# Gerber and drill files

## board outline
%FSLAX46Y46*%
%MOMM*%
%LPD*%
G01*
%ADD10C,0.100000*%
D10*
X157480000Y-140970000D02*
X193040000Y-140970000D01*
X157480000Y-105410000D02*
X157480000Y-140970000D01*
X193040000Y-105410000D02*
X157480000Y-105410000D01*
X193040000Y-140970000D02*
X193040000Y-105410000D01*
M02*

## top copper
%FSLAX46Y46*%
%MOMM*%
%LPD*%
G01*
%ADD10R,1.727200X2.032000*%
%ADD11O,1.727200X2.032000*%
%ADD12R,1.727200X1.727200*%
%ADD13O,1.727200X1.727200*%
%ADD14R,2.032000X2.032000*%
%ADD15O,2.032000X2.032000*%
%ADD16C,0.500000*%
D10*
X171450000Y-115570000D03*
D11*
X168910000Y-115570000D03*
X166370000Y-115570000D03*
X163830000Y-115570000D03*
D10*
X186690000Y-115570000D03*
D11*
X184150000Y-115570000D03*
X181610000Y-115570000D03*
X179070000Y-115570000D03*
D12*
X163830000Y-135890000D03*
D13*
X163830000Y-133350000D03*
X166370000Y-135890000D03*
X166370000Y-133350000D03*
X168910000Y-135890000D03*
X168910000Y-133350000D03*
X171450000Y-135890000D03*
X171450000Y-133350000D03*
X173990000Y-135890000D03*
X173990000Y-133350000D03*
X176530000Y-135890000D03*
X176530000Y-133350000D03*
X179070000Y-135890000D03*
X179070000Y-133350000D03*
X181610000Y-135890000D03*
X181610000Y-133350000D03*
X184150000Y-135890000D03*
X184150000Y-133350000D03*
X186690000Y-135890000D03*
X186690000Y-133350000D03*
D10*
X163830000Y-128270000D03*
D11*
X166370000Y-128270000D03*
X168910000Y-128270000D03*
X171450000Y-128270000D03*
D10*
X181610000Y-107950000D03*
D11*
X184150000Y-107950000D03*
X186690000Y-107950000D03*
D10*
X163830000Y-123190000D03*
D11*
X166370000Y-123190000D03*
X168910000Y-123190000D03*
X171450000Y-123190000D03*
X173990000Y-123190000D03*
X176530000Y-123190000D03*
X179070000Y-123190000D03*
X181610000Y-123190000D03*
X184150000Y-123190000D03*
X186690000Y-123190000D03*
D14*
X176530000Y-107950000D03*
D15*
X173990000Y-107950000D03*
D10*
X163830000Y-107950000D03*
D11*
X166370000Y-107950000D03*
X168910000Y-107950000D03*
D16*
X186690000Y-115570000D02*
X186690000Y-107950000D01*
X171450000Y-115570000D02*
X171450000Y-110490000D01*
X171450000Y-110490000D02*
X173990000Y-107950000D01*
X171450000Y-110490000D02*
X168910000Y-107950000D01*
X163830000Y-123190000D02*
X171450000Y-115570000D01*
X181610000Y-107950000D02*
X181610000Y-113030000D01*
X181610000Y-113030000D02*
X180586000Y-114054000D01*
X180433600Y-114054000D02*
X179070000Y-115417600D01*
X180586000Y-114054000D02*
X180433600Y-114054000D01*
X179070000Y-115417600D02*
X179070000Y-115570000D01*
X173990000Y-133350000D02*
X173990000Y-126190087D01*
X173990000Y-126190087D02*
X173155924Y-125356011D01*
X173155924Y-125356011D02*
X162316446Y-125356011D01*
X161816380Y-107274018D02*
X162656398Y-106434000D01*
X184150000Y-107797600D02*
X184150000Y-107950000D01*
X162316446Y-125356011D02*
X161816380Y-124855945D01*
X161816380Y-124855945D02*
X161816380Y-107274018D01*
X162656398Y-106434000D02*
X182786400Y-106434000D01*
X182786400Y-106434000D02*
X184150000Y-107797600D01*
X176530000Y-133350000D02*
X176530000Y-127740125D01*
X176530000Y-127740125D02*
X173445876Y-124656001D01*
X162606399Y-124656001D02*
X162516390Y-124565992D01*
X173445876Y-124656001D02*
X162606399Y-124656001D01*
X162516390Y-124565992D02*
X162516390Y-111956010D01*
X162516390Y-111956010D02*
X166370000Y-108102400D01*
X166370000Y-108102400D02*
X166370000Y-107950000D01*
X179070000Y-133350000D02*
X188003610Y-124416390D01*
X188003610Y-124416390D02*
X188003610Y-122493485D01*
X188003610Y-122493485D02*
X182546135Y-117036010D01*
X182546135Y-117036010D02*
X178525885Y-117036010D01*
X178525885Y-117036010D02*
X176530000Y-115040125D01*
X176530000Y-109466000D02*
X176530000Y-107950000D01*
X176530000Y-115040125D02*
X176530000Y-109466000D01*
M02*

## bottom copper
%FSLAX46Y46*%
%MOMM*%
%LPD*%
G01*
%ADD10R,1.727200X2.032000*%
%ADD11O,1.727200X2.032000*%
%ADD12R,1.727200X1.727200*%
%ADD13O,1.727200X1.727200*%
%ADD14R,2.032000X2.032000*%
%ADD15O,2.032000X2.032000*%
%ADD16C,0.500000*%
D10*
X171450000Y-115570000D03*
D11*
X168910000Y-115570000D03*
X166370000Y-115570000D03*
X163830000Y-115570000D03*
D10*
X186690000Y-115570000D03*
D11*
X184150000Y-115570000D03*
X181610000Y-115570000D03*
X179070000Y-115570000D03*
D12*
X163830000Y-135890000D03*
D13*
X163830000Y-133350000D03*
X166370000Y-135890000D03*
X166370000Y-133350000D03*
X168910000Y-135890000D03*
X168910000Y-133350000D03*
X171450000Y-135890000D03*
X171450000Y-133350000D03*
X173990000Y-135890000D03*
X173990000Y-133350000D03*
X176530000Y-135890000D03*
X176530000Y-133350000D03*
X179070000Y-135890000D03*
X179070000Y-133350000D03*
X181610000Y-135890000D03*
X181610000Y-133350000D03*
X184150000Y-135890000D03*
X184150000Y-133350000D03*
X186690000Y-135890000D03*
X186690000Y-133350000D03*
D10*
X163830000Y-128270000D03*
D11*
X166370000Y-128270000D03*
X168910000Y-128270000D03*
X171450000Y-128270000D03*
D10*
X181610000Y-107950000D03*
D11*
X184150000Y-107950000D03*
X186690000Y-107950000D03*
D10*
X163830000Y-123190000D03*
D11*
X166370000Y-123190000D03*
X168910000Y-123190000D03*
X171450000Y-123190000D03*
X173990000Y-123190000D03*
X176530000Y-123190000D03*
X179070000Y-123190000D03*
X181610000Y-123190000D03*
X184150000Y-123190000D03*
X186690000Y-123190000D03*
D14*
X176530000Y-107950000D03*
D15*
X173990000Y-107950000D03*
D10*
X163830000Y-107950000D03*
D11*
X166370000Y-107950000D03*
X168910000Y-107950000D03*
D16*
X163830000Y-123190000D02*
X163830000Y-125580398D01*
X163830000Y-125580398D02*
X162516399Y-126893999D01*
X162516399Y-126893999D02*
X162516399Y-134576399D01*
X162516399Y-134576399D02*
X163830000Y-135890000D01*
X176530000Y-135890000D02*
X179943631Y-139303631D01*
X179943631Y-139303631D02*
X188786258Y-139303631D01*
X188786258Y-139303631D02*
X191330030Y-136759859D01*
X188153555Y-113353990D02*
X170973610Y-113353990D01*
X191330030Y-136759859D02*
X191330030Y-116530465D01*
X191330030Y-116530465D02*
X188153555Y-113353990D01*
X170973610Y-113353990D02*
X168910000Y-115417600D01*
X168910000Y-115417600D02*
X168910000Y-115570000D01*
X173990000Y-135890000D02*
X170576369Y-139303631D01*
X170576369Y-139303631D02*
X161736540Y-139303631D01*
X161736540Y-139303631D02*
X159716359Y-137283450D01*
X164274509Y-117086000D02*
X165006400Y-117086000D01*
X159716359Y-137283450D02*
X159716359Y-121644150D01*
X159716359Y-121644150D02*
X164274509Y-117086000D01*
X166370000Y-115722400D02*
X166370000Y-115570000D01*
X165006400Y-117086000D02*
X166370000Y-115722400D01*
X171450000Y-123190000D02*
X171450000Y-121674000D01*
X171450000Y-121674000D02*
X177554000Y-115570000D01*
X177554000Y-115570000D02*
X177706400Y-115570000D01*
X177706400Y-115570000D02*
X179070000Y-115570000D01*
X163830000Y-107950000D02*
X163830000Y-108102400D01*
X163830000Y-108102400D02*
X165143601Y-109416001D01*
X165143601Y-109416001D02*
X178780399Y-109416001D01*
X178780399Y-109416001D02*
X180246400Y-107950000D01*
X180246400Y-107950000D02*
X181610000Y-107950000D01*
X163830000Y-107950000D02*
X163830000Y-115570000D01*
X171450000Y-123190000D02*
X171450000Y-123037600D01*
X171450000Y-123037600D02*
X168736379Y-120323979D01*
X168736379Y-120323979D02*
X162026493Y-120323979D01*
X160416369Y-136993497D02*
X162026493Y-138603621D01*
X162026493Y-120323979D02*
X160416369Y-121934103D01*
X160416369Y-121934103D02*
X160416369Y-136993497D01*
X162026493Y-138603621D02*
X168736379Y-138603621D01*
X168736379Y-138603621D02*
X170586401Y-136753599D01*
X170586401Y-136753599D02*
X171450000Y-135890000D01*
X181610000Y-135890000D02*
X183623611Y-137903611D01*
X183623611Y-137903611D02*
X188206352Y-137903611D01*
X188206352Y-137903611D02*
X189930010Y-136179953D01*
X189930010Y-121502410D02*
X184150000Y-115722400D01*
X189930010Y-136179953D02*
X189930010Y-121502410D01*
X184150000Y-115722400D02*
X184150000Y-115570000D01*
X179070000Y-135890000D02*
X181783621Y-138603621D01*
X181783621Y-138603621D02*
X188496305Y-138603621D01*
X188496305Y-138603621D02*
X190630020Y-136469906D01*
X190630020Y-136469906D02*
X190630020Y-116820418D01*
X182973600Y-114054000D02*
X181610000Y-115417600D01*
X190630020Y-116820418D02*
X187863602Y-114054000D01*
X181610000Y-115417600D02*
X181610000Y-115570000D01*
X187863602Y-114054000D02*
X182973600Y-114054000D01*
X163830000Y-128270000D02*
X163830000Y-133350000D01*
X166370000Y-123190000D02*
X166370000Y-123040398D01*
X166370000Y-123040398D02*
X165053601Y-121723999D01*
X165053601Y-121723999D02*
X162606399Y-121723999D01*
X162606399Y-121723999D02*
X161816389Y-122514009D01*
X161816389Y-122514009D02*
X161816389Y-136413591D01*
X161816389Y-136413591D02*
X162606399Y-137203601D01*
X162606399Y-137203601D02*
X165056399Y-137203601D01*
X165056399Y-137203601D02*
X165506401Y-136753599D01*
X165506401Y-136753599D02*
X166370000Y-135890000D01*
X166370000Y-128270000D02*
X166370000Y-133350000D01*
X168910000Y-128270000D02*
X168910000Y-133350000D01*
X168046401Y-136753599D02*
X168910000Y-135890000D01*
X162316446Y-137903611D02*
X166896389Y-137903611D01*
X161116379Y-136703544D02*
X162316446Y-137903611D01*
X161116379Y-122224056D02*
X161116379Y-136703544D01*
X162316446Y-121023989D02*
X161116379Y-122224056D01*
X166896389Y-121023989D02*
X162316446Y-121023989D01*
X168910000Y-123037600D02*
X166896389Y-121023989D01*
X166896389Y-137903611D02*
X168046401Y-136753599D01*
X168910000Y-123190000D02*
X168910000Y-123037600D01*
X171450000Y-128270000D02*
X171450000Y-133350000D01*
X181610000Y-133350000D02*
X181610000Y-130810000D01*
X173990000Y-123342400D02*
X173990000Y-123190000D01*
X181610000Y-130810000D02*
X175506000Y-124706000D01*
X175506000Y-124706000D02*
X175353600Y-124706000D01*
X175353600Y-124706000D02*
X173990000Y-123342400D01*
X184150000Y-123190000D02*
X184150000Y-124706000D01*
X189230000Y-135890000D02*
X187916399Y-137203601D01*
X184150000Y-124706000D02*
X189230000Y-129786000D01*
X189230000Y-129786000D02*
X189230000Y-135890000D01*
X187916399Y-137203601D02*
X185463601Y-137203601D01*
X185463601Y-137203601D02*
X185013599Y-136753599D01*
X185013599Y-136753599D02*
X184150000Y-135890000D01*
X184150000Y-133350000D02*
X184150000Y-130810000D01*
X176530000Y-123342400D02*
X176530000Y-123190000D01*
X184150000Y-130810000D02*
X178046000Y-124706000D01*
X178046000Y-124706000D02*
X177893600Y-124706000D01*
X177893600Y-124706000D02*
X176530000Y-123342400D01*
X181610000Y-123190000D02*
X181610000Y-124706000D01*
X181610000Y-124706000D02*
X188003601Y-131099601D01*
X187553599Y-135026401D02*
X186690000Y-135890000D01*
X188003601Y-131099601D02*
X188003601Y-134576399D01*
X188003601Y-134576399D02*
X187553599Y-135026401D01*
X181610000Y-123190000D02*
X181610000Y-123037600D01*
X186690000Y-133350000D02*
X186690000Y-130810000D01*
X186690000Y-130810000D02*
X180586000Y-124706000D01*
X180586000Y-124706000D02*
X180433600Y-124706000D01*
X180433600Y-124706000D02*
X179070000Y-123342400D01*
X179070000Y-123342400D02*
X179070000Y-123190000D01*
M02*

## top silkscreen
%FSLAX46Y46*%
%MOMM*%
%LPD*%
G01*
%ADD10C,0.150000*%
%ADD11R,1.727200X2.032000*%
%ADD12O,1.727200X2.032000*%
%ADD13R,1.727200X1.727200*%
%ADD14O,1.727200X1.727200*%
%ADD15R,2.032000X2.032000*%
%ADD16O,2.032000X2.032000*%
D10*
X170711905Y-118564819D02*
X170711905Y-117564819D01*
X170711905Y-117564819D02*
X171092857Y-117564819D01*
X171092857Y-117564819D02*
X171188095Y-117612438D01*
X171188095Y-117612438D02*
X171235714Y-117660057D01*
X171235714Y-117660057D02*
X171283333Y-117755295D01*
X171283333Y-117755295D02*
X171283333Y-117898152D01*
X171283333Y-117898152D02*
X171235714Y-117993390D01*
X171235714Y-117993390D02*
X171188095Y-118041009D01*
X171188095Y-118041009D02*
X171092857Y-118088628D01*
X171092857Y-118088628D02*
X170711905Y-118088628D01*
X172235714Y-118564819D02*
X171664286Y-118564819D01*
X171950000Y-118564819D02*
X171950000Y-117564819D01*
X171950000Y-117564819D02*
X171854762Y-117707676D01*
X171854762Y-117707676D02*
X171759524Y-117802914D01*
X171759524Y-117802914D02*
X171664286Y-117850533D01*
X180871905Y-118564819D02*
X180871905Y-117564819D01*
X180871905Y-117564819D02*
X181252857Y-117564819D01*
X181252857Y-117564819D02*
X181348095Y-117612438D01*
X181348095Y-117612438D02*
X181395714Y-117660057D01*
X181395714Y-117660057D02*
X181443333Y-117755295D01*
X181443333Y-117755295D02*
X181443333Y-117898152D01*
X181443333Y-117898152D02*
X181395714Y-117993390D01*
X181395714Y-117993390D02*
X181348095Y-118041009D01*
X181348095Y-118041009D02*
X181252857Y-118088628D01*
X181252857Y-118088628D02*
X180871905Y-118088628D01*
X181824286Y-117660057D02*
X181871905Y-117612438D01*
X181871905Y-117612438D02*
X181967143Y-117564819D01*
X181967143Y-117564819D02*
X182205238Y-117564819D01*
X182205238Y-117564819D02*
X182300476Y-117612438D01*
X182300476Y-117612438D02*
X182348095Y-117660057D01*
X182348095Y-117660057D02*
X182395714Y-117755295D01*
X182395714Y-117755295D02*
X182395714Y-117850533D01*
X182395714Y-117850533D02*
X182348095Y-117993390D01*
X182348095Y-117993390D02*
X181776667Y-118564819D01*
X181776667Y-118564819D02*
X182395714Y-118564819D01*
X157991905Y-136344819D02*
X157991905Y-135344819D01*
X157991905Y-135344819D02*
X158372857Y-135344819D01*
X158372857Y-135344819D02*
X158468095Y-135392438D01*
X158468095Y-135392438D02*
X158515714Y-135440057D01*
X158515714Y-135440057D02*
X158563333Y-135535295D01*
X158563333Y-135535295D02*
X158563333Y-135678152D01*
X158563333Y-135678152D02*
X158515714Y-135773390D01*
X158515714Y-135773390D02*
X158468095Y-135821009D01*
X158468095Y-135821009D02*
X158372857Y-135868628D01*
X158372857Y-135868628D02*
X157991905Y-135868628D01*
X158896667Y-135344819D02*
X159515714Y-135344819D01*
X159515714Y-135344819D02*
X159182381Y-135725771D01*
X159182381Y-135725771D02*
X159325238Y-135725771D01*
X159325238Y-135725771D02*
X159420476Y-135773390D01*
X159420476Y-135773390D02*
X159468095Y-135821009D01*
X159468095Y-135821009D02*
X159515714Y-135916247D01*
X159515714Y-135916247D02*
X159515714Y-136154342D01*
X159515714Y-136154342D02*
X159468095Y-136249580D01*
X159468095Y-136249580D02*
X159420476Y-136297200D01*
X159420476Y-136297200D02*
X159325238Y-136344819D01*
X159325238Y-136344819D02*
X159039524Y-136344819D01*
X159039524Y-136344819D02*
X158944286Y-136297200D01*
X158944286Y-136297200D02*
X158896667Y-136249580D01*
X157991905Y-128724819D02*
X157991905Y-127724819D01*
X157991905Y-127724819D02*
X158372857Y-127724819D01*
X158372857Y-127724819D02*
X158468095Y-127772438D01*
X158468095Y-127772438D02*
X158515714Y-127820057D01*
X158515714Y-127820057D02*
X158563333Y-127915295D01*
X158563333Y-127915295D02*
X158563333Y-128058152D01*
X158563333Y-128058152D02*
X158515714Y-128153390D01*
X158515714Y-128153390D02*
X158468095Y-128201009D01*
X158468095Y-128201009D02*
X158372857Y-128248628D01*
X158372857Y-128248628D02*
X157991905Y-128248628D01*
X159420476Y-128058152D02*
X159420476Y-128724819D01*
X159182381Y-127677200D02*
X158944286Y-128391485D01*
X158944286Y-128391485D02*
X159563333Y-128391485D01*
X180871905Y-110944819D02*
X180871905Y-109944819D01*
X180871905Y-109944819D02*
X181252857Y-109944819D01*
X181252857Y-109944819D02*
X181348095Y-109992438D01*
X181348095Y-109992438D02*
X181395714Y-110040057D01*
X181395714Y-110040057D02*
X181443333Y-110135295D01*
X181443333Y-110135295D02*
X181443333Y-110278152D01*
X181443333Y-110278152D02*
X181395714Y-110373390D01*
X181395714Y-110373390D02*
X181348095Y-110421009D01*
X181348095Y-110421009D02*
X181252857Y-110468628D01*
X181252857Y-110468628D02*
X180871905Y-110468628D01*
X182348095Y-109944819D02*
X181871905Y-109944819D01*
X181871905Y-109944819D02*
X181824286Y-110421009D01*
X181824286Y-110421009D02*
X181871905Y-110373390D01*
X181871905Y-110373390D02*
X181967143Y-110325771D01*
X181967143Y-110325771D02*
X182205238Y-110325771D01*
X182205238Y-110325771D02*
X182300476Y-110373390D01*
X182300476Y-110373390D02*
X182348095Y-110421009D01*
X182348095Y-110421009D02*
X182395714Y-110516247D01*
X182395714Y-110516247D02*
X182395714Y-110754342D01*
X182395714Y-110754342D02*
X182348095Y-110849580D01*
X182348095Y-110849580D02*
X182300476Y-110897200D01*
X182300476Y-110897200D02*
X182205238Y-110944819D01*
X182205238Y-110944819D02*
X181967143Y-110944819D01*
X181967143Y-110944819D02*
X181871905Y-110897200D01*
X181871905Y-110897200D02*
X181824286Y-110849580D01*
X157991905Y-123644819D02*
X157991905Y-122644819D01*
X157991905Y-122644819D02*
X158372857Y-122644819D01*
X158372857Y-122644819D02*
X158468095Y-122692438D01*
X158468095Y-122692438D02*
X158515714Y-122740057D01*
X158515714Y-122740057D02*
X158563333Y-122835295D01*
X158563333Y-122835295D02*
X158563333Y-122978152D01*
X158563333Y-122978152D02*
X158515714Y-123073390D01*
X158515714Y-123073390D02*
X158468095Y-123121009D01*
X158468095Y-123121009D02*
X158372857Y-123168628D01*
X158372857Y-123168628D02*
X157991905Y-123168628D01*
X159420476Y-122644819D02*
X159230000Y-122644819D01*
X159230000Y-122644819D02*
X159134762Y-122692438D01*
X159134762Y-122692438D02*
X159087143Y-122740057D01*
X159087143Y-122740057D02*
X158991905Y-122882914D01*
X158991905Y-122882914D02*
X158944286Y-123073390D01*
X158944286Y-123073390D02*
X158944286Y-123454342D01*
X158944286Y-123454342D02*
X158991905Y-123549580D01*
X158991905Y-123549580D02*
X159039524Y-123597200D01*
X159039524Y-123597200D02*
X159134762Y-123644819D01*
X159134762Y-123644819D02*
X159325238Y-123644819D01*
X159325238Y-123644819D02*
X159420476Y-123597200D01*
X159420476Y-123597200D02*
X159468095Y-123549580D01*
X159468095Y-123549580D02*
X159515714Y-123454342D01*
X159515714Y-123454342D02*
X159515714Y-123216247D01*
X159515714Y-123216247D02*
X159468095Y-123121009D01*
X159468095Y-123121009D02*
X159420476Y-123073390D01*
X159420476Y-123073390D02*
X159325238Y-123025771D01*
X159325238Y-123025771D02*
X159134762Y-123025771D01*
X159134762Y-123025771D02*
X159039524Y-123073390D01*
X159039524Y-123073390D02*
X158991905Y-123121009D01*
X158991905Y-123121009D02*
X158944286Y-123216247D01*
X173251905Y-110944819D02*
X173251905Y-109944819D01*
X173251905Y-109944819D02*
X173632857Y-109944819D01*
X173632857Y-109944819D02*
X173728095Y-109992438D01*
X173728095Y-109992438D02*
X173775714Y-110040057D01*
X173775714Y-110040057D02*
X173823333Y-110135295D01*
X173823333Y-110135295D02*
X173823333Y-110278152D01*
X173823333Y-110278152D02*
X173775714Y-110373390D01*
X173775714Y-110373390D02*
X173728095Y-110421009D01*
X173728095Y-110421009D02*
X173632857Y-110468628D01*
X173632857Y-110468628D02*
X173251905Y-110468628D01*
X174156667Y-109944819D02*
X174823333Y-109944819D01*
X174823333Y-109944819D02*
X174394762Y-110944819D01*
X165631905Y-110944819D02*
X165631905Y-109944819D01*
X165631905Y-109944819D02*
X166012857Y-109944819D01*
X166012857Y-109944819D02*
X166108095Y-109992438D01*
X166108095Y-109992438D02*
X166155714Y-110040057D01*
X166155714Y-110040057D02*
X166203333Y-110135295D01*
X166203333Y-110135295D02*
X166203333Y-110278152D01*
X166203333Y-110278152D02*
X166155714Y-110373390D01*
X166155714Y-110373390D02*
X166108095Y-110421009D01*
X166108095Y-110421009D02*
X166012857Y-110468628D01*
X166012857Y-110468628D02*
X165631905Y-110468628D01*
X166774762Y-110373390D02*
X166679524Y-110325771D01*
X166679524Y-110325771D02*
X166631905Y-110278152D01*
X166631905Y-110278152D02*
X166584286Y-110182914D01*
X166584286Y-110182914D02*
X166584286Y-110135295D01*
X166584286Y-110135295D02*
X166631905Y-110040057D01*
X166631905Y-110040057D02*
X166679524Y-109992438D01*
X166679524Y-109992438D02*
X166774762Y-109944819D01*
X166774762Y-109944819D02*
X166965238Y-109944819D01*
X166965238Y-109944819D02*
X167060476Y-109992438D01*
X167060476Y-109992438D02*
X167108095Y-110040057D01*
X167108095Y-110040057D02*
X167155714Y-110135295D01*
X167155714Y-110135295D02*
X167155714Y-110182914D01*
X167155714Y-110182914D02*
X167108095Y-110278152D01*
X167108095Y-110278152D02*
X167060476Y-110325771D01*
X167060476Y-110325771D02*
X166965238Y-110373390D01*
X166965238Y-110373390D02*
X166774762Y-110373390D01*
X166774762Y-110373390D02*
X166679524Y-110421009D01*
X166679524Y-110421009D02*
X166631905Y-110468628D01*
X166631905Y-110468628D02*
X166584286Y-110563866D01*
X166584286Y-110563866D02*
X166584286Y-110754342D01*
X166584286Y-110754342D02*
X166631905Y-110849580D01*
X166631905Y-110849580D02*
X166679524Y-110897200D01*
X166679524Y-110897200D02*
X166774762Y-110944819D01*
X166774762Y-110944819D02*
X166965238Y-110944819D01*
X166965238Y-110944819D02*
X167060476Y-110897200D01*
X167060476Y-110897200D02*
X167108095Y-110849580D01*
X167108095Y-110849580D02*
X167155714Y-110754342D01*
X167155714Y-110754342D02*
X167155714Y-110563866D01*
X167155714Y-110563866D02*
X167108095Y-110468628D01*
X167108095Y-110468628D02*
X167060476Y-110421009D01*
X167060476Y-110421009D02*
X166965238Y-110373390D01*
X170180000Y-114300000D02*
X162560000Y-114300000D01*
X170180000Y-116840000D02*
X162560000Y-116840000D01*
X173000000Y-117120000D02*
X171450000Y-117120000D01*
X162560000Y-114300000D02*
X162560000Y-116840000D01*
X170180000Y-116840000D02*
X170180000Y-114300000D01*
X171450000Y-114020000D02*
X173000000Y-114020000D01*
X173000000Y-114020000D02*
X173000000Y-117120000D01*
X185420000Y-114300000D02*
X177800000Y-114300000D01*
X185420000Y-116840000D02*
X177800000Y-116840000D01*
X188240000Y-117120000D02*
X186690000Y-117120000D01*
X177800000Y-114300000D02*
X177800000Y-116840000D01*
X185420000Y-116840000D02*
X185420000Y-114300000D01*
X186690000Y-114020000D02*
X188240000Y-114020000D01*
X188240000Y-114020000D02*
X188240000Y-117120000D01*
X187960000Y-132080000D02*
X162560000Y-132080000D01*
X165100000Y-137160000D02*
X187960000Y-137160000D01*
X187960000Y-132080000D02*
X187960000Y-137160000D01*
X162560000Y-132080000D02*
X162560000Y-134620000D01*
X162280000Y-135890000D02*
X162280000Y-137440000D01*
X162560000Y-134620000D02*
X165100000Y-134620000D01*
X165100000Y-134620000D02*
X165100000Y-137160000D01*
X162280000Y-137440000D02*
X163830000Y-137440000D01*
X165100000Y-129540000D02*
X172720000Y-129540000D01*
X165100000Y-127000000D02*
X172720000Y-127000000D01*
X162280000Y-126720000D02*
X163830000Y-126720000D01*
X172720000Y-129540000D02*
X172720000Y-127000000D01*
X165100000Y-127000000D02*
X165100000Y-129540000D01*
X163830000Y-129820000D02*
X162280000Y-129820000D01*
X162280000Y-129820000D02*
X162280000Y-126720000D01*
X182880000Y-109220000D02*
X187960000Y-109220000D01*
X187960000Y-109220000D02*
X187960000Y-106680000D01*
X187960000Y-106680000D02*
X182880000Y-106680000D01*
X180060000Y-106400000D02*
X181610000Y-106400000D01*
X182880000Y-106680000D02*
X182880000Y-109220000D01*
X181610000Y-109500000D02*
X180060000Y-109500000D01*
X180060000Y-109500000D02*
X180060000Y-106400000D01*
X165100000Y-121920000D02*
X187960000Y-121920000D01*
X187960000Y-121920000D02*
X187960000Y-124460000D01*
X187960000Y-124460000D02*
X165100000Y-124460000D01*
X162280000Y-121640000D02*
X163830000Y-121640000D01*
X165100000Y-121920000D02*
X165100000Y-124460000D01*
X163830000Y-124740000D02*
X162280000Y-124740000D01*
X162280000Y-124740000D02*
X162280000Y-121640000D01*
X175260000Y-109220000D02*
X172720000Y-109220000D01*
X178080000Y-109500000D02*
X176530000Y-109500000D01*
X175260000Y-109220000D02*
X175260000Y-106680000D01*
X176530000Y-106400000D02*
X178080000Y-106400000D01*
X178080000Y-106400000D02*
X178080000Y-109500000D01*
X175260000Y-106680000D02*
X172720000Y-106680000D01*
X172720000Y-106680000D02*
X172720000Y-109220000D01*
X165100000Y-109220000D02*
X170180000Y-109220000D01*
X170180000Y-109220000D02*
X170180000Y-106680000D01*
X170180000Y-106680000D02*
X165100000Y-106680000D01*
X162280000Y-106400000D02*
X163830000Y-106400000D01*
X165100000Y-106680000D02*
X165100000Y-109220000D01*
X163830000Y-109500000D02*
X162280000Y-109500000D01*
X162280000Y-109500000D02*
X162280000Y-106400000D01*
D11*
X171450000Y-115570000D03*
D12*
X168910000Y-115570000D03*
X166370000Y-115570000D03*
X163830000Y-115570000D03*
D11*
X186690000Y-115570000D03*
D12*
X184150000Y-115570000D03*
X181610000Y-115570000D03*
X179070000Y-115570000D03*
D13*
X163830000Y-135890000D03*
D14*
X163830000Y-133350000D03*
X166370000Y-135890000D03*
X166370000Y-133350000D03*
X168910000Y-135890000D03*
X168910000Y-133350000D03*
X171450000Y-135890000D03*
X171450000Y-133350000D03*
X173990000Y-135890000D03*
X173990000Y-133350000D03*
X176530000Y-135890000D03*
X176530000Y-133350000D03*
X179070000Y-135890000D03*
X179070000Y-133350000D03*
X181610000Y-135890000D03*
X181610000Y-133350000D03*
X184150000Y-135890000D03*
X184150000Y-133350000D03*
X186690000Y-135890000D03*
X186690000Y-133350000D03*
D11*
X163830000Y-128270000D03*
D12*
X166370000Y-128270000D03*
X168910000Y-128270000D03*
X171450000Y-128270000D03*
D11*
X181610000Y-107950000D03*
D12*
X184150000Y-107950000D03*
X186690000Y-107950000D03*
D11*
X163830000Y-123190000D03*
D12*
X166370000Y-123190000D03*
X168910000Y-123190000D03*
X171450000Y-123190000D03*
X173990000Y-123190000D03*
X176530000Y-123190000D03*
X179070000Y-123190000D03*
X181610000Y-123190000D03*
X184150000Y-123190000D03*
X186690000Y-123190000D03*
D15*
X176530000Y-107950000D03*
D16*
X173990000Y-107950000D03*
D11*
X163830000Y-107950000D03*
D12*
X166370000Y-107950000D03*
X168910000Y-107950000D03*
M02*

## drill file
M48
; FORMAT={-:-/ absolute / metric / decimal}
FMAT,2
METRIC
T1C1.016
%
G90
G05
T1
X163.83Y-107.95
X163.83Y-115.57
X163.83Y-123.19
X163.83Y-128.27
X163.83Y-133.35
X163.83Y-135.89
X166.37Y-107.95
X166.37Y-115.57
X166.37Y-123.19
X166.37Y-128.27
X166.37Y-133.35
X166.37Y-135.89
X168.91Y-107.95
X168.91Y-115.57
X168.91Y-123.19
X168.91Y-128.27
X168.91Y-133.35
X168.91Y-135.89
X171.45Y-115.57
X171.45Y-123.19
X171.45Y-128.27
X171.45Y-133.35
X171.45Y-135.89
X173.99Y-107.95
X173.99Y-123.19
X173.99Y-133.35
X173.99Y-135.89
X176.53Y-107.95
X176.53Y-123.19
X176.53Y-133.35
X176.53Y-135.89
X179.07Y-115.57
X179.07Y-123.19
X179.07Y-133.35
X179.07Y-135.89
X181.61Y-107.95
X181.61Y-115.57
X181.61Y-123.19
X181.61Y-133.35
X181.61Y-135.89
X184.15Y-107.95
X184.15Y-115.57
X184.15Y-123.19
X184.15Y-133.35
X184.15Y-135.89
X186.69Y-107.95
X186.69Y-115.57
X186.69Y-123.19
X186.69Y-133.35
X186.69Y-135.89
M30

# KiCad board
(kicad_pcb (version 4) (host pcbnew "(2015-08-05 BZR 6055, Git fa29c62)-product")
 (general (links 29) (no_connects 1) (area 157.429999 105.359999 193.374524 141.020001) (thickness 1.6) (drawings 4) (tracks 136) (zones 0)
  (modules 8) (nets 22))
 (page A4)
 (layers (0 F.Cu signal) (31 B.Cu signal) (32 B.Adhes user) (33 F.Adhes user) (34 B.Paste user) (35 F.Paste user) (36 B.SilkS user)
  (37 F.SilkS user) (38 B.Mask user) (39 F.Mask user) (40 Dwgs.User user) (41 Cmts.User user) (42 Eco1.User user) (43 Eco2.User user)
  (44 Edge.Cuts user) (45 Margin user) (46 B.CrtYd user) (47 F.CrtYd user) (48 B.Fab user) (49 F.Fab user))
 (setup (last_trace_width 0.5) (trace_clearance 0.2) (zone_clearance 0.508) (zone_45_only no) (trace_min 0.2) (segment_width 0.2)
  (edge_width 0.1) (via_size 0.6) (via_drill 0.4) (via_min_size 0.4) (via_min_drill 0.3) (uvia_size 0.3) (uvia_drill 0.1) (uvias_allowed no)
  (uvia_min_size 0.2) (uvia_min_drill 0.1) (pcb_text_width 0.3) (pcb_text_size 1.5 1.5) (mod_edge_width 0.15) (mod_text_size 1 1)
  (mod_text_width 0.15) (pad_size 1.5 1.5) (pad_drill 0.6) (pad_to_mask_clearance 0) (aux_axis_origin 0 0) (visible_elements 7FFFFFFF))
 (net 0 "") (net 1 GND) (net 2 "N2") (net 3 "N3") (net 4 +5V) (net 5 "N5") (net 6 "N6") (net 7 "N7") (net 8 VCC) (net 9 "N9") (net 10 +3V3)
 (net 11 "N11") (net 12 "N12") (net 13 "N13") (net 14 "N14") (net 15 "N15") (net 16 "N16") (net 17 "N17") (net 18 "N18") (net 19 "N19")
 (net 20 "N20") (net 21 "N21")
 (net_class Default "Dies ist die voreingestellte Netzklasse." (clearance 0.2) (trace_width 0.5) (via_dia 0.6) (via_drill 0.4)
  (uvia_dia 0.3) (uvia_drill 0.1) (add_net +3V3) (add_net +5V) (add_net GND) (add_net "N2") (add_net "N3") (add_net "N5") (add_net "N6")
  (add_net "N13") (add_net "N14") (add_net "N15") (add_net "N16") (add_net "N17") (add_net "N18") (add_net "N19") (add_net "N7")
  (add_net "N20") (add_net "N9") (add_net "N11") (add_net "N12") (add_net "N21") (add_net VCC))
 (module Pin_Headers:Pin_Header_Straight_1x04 (layer F.Cu) (at 171.45 115.57 270)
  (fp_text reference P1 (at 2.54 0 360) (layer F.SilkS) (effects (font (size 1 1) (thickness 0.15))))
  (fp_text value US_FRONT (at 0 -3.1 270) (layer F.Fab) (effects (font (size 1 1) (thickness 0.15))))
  (fp_line (start -1.27 1.27) (end -1.27 8.89) (layer F.SilkS) (width 0.15))
  (fp_line (start 1.27 1.27) (end 1.27 8.89) (layer F.SilkS) (width 0.15))
  (fp_line (start 1.55 -1.55) (end 1.55 0) (layer F.SilkS) (width 0.15))
  (fp_line (start -1.27 8.89) (end 1.27 8.89) (layer F.SilkS) (width 0.15))
  (fp_line (start 1.27 1.27) (end -1.27 1.27) (layer F.SilkS) (width 0.15))
  (fp_line (start -1.55 0) (end -1.55 -1.55) (layer F.SilkS) (width 0.15))
  (fp_line (start -1.55 -1.55) (end 1.55 -1.55) (layer F.SilkS) (width 0.15))
  (pad 1 thru_hole rect (at 0 0 270) (size 2.032 1.7272) (drill 1.016) (layers *.Cu *.Mask F.SilkS) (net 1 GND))
  (pad 2 thru_hole oval (at 0 2.54 270) (size 2.032 1.7272) (drill 1.016) (layers *.Cu *.Mask F.SilkS) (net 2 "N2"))
  (pad 3 thru_hole oval (at 0 5.08 270) (size 2.032 1.7272) (drill 1.016) (layers *.Cu *.Mask F.SilkS) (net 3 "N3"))
  (pad 4 thru_hole oval (at 0 7.62 270) (size 2.032 1.7272) (drill 1.016) (layers *.Cu *.Mask F.SilkS) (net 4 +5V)))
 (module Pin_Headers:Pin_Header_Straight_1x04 (layer F.Cu) (at 186.69 115.57 270)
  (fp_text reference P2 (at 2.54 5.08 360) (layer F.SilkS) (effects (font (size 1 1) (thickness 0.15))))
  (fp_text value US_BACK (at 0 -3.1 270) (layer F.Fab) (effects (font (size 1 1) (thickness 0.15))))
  (fp_line (start -1.27 1.27) (end -1.27 8.89) (layer F.SilkS) (width 0.15))
  (fp_line (start 1.27 1.27) (end 1.27 8.89) (layer F.SilkS) (width 0.15))
  (fp_line (start 1.55 -1.55) (end 1.55 0) (layer F.SilkS) (width 0.15))
  (fp_line (start -1.27 8.89) (end 1.27 8.89) (layer F.SilkS) (width 0.15))
  (fp_line (start 1.27 1.27) (end -1.27 1.27) (layer F.SilkS) (width 0.15))
  (fp_line (start -1.55 0) (end -1.55 -1.55) (layer F.SilkS) (width 0.15))
  (fp_line (start -1.55 -1.55) (end 1.55 -1.55) (layer F.SilkS) (width 0.15))
  (pad 1 thru_hole rect (at 0 0 270) (size 2.032 1.7272) (drill 1.016) (layers *.Cu *.Mask F.SilkS) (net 1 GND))
  (pad 2 thru_hole oval (at 0 2.54 270) (size 2.032 1.7272) (drill 1.016) (layers *.Cu *.Mask F.SilkS) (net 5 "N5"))
  (pad 3 thru_hole oval (at 0 5.08 270) (size 2.032 1.7272) (drill 1.016) (layers *.Cu *.Mask F.SilkS) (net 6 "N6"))
  (pad 4 thru_hole oval (at 0 7.62 270) (size 2.032 1.7272) (drill 1.016) (layers *.Cu *.Mask F.SilkS) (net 4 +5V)))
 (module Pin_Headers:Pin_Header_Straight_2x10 (layer F.Cu) (at 163.83 135.89 90)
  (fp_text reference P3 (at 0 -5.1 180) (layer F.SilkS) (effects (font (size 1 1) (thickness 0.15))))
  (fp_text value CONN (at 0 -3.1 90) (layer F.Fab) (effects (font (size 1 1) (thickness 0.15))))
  (fp_line (start 3.81 24.13) (end 3.81 -1.27) (layer F.SilkS) (width 0.15))
  (fp_line (start -1.27 1.27) (end -1.27 24.13) (layer F.SilkS) (width 0.15))
  (fp_line (start 3.81 24.13) (end -1.27 24.13) (layer F.SilkS) (width 0.15))
  (fp_line (start 3.81 -1.27) (end 1.27 -1.27) (layer F.SilkS) (width 0.15))
  (fp_line (start 0 -1.55) (end -1.55 -1.55) (layer F.SilkS) (width 0.15))
  (fp_line (start 1.27 -1.27) (end 1.27 1.27) (layer F.SilkS) (width 0.15))
  (fp_line (start 1.27 1.27) (end -1.27 1.27) (layer F.SilkS) (width 0.15))
  (fp_line (start -1.55 -1.55) (end -1.55 0) (layer F.SilkS) (width 0.15))
  (pad 1 thru_hole rect (at 0 0 90) (size 1.7272 1.7272) (drill 1.016) (layers *.Cu *.Mask F.SilkS) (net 1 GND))
  (pad 2 thru_hole oval (at 2.54 0 90) (size 1.7272 1.7272) (drill 1.016) (layers *.Cu *.Mask F.SilkS) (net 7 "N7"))
  (pad 3 thru_hole oval (at 0 2.54 90) (size 1.7272 1.7272) (drill 1.016) (layers *.Cu *.Mask F.SilkS) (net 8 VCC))
  (pad 4 thru_hole oval (at 2.54 2.54 90) (size 1.7272 1.7272) (drill 1.016) (layers *.Cu *.Mask F.SilkS) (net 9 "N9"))
  (pad 5 thru_hole oval (at 0 5.08 90) (size 1.7272 1.7272) (drill 1.016) (layers *.Cu *.Mask F.SilkS) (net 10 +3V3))
  (pad 6 thru_hole oval (at 2.54 5.08 90) (size 1.7272 1.7272) (drill 1.016) (layers *.Cu *.Mask F.SilkS) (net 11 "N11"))
  (pad 7 thru_hole oval (at 0 7.62 90) (size 1.7272 1.7272) (drill 1.016) (layers *.Cu *.Mask F.SilkS) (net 4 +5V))
  (pad 8 thru_hole oval (at 2.54 7.62 90) (size 1.7272 1.7272) (drill 1.016) (layers *.Cu *.Mask F.SilkS) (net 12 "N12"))
  (pad 9 thru_hole oval (at 0 10.16 90) (size 1.7272 1.7272) (drill 1.016) (layers *.Cu *.Mask F.SilkS) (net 3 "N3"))
  (pad 10 thru_hole oval (at 2.54 10.16 90) (size 1.7272 1.7272) (drill 1.016) (layers *.Cu *.Mask F.SilkS) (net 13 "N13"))
  (pad 11 thru_hole oval (at 0 12.7 90) (size 1.7272 1.7272) (drill 1.016) (layers *.Cu *.Mask F.SilkS) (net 2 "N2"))
  (pad 12 thru_hole oval (at 2.54 12.7 90) (size 1.7272 1.7272) (drill 1.016) (layers *.Cu *.Mask F.SilkS) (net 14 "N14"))
  (pad 13 thru_hole oval (at 0 15.24 90) (size 1.7272 1.7272) (drill 1.016) (layers *.Cu *.Mask F.SilkS) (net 6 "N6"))
  (pad 14 thru_hole oval (at 2.54 15.24 90) (size 1.7272 1.7272) (drill 1.016) (layers *.Cu *.Mask F.SilkS) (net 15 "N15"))
  (pad 15 thru_hole oval (at 0 17.78 90) (size 1.7272 1.7272) (drill 1.016) (layers *.Cu *.Mask F.SilkS) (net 5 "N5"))
  (pad 16 thru_hole oval (at 2.54 17.78 90) (size 1.7272 1.7272) (drill 1.016) (layers *.Cu *.Mask F.SilkS) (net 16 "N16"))
  (pad 17 thru_hole oval (at 0 20.32 90) (size 1.7272 1.7272) (drill 1.016) (layers *.Cu *.Mask F.SilkS) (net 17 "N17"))
  (pad 18 thru_hole oval (at 2.54 20.32 90) (size 1.7272 1.7272) (drill 1.016) (layers *.Cu *.Mask F.SilkS) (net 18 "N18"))
  (pad 19 thru_hole oval (at 0 22.86 90) (size 1.7272 1.7272) (drill 1.016) (layers *.Cu *.Mask F.SilkS) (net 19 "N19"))
  (pad 20 thru_hole oval (at 2.54 22.86 90) (size 1.7272 1.7272) (drill 1.016) (layers *.Cu *.Mask F.SilkS) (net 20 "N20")))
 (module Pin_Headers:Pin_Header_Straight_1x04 (layer F.Cu) (at 163.83 128.27 90)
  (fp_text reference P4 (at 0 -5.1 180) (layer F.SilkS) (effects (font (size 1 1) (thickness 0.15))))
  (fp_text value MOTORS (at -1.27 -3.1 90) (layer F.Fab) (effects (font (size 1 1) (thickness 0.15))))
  (fp_line (start -1.27 1.27) (end -1.27 8.89) (layer F.SilkS) (width 0.15))
  (fp_line (start 1.27 1.27) (end 1.27 8.89) (layer F.SilkS) (width 0.15))
  (fp_line (start 1.55 -1.55) (end 1.55 0) (layer F.SilkS) (width 0.15))
  (fp_line (start -1.27 8.89) (end 1.27 8.89) (layer F.SilkS) (width 0.15))
  (fp_line (start 1.27 1.27) (end -1.27 1.27) (layer F.SilkS) (width 0.15))
  (fp_line (start -1.55 0) (end -1.55 -1.55) (layer F.SilkS) (width 0.15))
  (fp_line (start -1.55 -1.55) (end 1.55 -1.55) (layer F.SilkS) (width 0.15))
  (pad 1 thru_hole rect (at 0 0 90) (size 2.032 1.7272) (drill 1.016) (layers *.Cu *.Mask F.SilkS) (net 7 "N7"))
  (pad 2 thru_hole oval (at 0 2.54 90) (size 2.032 1.7272) (drill 1.016) (layers *.Cu *.Mask F.SilkS) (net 9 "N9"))
  (pad 3 thru_hole oval (at 0 5.08 90) (size 2.032 1.7272) (drill 1.016) (layers *.Cu *.Mask F.SilkS) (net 11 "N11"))
  (pad 4 thru_hole oval (at 0 7.62 90) (size 2.032 1.7272) (drill 1.016) (layers *.Cu *.Mask F.SilkS) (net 12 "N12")))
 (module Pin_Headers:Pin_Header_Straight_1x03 (layer F.Cu) (at 181.61 107.95 90)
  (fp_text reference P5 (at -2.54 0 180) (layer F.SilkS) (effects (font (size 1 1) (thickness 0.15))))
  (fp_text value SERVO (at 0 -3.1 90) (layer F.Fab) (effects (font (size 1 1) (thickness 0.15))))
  (fp_line (start -1.27 1.27) (end -1.27 6.35) (layer F.SilkS) (width 0.15))
  (fp_line (start -1.27 6.35) (end 1.27 6.35) (layer F.SilkS) (width 0.15))
  (fp_line (start 1.27 6.35) (end 1.27 1.27) (layer F.SilkS) (width 0.15))
  (fp_line (start 1.55 -1.55) (end 1.55 0) (layer F.SilkS) (width 0.15))
  (fp_line (start 1.27 1.27) (end -1.27 1.27) (layer F.SilkS) (width 0.15))
  (fp_line (start -1.55 0) (end -1.55 -1.55) (layer F.SilkS) (width 0.15))
  (fp_line (start -1.55 -1.55) (end 1.55 -1.55) (layer F.SilkS) (width 0.15))
  (pad 1 thru_hole rect (at 0 0 90) (size 2.032 1.7272) (drill 1.016) (layers *.Cu *.Mask F.SilkS) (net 4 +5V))
  (pad 2 thru_hole oval (at 0 2.54 90) (size 2.032 1.7272) (drill 1.016) (layers *.Cu *.Mask F.SilkS) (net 13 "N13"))
  (pad 3 thru_hole oval (at 0 5.08 90) (size 2.032 1.7272) (drill 1.016) (layers *.Cu *.Mask F.SilkS) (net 1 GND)))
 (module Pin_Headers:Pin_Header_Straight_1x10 (layer F.Cu) (at 163.83 123.19 90)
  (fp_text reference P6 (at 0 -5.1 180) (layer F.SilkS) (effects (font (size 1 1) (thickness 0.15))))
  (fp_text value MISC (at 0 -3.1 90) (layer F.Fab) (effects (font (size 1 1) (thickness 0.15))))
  (fp_line (start 1.27 1.27) (end 1.27 24.13) (layer F.SilkS) (width 0.15))
  (fp_line (start 1.27 24.13) (end -1.27 24.13) (layer F.SilkS) (width 0.15))
  (fp_line (start -1.27 24.13) (end -1.27 1.27) (layer F.SilkS) (width 0.15))
  (fp_line (start 1.55 -1.55) (end 1.55 0) (layer F.SilkS) (width 0.15))
  (fp_line (start 1.27 1.27) (end -1.27 1.27) (layer F.SilkS) (width 0.15))
  (fp_line (start -1.55 0) (end -1.55 -1.55) (layer F.SilkS) (width 0.15))
  (fp_line (start -1.55 -1.55) (end 1.55 -1.55) (layer F.SilkS) (width 0.15))
  (pad 1 thru_hole rect (at 0 0 90) (size 2.032 1.7272) (drill 1.016) (layers *.Cu *.Mask F.SilkS) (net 1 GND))
  (pad 2 thru_hole oval (at 0 2.54 90) (size 2.032 1.7272) (drill 1.016) (layers *.Cu *.Mask F.SilkS) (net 8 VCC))
  (pad 3 thru_hole oval (at 0 5.08 90) (size 2.032 1.7272) (drill 1.016) (layers *.Cu *.Mask F.SilkS) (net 10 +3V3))
  (pad 4 thru_hole oval (at 0 7.62 90) (size 2.032 1.7272) (drill 1.016) (layers *.Cu *.Mask F.SilkS) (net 4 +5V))
  (pad 5 thru_hole oval (at 0 10.16 90) (size 2.032 1.7272) (drill 1.016) (layers *.Cu *.Mask F.SilkS) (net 16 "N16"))
  (pad 6 thru_hole oval (at 0 12.7 90) (size 2.032 1.7272) (drill 1.016) (layers *.Cu *.Mask F.SilkS) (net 18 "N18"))
  (pad 7 thru_hole oval (at 0 15.24 90) (size 2.032 1.7272) (drill 1.016) (layers *.Cu *.Mask F.SilkS) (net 20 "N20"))
  (pad 8 thru_hole oval (at 0 17.78 90) (size 2.032 1.7272) (drill 1.016) (layers *.Cu *.Mask F.SilkS) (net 19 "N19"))
  (pad 9 thru_hole oval (at 0 20.32 90) (size 2.032 1.7272) (drill 1.016) (layers *.Cu *.Mask F.SilkS) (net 17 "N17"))
  (pad 10 thru_hole oval (at 0 22.86 90) (size 2.032 1.7272) (drill 1.016) (layers *.Cu *.Mask F.SilkS) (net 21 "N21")))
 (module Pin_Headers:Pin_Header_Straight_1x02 (layer F.Cu) (at 176.53 107.95 270)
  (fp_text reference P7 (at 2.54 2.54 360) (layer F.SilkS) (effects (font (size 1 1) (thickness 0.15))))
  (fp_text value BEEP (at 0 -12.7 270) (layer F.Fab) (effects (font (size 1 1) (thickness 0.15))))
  (fp_line (start 1.27 1.27) (end 1.27 3.81) (layer F.SilkS) (width 0.15))
  (fp_line (start 1.55 -1.55) (end 1.55 0) (layer F.SilkS) (width 0.15))
  (fp_line (start 1.27 1.27) (end -1.27 1.27) (layer F.SilkS) (width 0.15))
  (fp_line (start -1.55 0) (end -1.55 -1.55) (layer F.SilkS) (width 0.15))
  (fp_line (start -1.55 -1.55) (end 1.55 -1.55) (layer F.SilkS) (width 0.15))
  (fp_line (start -1.27 1.27) (end -1.27 3.81) (layer F.SilkS) (width 0.15))
  (fp_line (start -1.27 3.81) (end 1.27 3.81) (layer F.SilkS) (width 0.15))
  (pad 1 thru_hole rect (at 0 0 270) (size 2.032 2.032) (drill 1.016) (layers *.Cu *.Mask F.SilkS) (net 15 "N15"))
  (pad 2 thru_hole oval (at 0 2.54 270) (size 2.032 2.032) (drill 1.016) (layers *.Cu *.Mask F.SilkS) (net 1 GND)))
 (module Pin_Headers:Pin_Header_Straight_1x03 (layer F.Cu) (at 163.83 107.95 90)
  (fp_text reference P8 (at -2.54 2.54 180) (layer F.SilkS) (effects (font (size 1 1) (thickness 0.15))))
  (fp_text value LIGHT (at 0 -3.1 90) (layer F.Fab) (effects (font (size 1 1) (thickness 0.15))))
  (fp_line (start -1.27 1.27) (end -1.27 6.35) (layer F.SilkS) (width 0.15))
  (fp_line (start -1.27 6.35) (end 1.27 6.35) (layer F.SilkS) (width 0.15))
  (fp_line (start 1.27 6.35) (end 1.27 1.27) (layer F.SilkS) (width 0.15))
  (fp_line (start 1.55 -1.55) (end 1.55 0) (layer F.SilkS) (width 0.15))
  (fp_line (start 1.27 1.27) (end -1.27 1.27) (layer F.SilkS) (width 0.15))
  (fp_line (start -1.55 0) (end -1.55 -1.55) (layer F.SilkS) (width 0.15))
  (fp_line (start -1.55 -1.55) (end 1.55 -1.55) (layer F.SilkS) (width 0.15))
  (pad 1 thru_hole rect (at 0 0 90) (size 2.032 1.7272) (drill 1.016) (layers *.Cu *.Mask F.SilkS) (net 4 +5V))
  (pad 2 thru_hole oval (at 0 2.54 90) (size 2.032 1.7272) (drill 1.016) (layers *.Cu *.Mask F.SilkS) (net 14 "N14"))
  (pad 3 thru_hole oval (at 0 5.08 90) (size 2.032 1.7272) (drill 1.016) (layers *.Cu *.Mask F.SilkS) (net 1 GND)))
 (gr_line (start 157.48 140.97) (end 193.04 140.97) (angle 90) (layer Edge.Cuts) (width 0.1))
 (gr_line (start 157.48 105.41) (end 157.48 140.97) (angle 90) (layer Edge.Cuts) (width 0.1))
 (gr_line (start 193.04 105.41) (end 157.48 105.41) (angle 90) (layer Edge.Cuts) (width 0.1))
 (gr_line (start 193.04 140.97) (end 193.04 105.41) (angle 90) (layer Edge.Cuts) (width 0.1))
 (segment (start 186.69 115.57) (end 186.69 107.95) (width 0.5) (layer F.Cu) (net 1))
 (segment (start 171.45 115.57) (end 171.45 110.49) (width 0.5) (layer F.Cu) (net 1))
 (segment (start 171.45 110.49) (end 173.99 107.95) (width 0.5) (layer F.Cu) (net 1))
 (segment (start 171.45 110.49) (end 168.91 107.95) (width 0.5) (layer F.Cu) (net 1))
 (segment (start 163.83 123.19) (end 171.45 115.57) (width 0.5) (layer F.Cu) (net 1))
 (segment (start 163.83 123.19) (end 163.83 125.580398) (width 0.5) (layer B.Cu) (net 1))
 (segment (start 163.83 125.580398) (end 162.516399 126.893999) (width 0.5) (layer B.Cu) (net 1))
 (segment (start 162.516399 126.893999) (end 162.516399 134.576399) (width 0.5) (layer B.Cu) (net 1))
 (segment (start 162.516399 134.576399) (end 163.83 135.89) (width 0.5) (layer B.Cu) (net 1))
 (segment (start 176.53 135.89) (end 179.943631 139.303631) (width 0.5) (layer B.Cu) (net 2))
 (segment (start 179.943631 139.303631) (end 188.786258 139.303631) (width 0.5) (layer B.Cu) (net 2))
 (segment (start 188.786258 139.303631) (end 191.33003 136.759859) (width 0.5) (layer B.Cu) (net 2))
 (segment (start 188.153555 113.35399) (end 170.97361 113.35399) (width 0.5) (layer B.Cu) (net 2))
 (segment (start 191.33003 136.759859) (end 191.33003 116.530465) (width 0.5) (layer B.Cu) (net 2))
 (segment (start 191.33003 116.530465) (end 188.153555 113.35399) (width 0.5) (layer B.Cu) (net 2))
 (segment (start 170.97361 113.35399) (end 168.91 115.4176) (width 0.5) (layer B.Cu) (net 2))
 (segment (start 168.91 115.4176) (end 168.91 115.57) (width 0.5) (layer B.Cu) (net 2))
 (segment (start 173.99 135.89) (end 170.576369 139.303631) (width 0.5) (layer B.Cu) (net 3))
 (segment (start 170.576369 139.303631) (end 161.73654 139.303631) (width 0.5) (layer B.Cu) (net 3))
 (segment (start 161.73654 139.303631) (end 159.716359 137.28345) (width 0.5) (layer B.Cu) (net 3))
 (segment (start 164.274509 117.086) (end 165.0064 117.086) (width 0.5) (layer B.Cu) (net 3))
 (segment (start 159.716359 137.28345) (end 159.716359 121.64415) (width 0.5) (layer B.Cu) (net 3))
 (segment (start 159.716359 121.64415) (end 164.274509 117.086) (width 0.5) (layer B.Cu) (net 3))
 (segment (start 166.37 115.7224) (end 166.37 115.57) (width 0.5) (layer B.Cu) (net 3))
 (segment (start 165.0064 117.086) (end 166.37 115.7224) (width 0.5) (layer B.Cu) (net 3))
 (segment (start 171.45 123.19) (end 171.45 121.674) (width 0.5) (layer B.Cu) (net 4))
 (segment (start 171.45 121.674) (end 177.554 115.57) (width 0.5) (layer B.Cu) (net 4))
 (segment (start 177.554 115.57) (end 177.7064 115.57) (width 0.5) (layer B.Cu) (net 4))
 (segment (start 177.7064 115.57) (end 179.07 115.57) (width 0.5) (layer B.Cu) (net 4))
 (segment (start 163.83 107.95) (end 163.83 108.1024) (width 0.5) (layer B.Cu) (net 4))
 (segment (start 163.83 108.1024) (end 165.143601 109.416001) (width 0.5) (layer B.Cu) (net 4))
 (segment (start 165.143601 109.416001) (end 178.780399 109.416001) (width 0.5) (layer B.Cu) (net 4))
 (segment (start 178.780399 109.416001) (end 180.2464 107.95) (width 0.5) (layer B.Cu) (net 4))
 (segment (start 180.2464 107.95) (end 181.61 107.95) (width 0.5) (layer B.Cu) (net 4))
 (segment (start 163.83 107.95) (end 163.83 115.57) (width 0.5) (layer B.Cu) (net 4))
 (segment (start 181.61 107.95) (end 181.61 113.03) (width 0.5) (layer F.Cu) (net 4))
 (segment (start 181.61 113.03) (end 180.586 114.054) (width 0.5) (layer F.Cu) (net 4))
 (segment (start 180.4336 114.054) (end 179.07 115.4176) (width 0.5) (layer F.Cu) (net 4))
 (segment (start 180.586 114.054) (end 180.4336 114.054) (width 0.5) (layer F.Cu) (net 4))
 (segment (start 179.07 115.4176) (end 179.07 115.57) (width 0.5) (layer F.Cu) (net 4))
 (segment (start 171.45 123.19) (end 171.45 123.0376) (width 0.5) (layer B.Cu) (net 4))
 (segment (start 171.45 123.0376) (end 168.736379 120.323979) (width 0.5) (layer B.Cu) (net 4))
 (segment (start 168.736379 120.323979) (end 162.026493 120.323979) (width 0.5) (layer B.Cu) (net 4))
 (segment (start 160.416369 136.993497) (end 162.026493 138.603621) (width 0.5) (layer B.Cu) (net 4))
 (segment (start 162.026493 120.323979) (end 160.416369 121.934103) (width 0.5) (layer B.Cu) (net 4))
 (segment (start 160.416369 121.934103) (end 160.416369 136.993497) (width 0.5) (layer B.Cu) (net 4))
 (segment (start 162.026493 138.603621) (end 168.736379 138.603621) (width 0.5) (layer B.Cu) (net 4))
 (segment (start 168.736379 138.603621) (end 170.586401 136.753599) (width 0.5) (layer B.Cu) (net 4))
 (segment (start 170.586401 136.753599) (end 171.45 135.89) (width 0.5) (layer B.Cu) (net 4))
 (segment (start 181.61 135.89) (end 183.623611 137.903611) (width 0.5) (layer B.Cu) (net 5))
 (segment (start 183.623611 137.903611) (end 188.206352 137.903611) (width 0.5) (layer B.Cu) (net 5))
 (segment (start 188.206352 137.903611) (end 189.93001 136.179953) (width 0.5) (layer B.Cu) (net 5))
 (segment (start 189.93001 121.50241) (end 184.15 115.7224) (width 0.5) (layer B.Cu) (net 5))
 (segment (start 189.93001 136.179953) (end 189.93001 121.50241) (width 0.5) (layer B.Cu) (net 5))
 (segment (start 184.15 115.7224) (end 184.15 115.57) (width 0.5) (layer B.Cu) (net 5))
 (segment (start 179.07 135.89) (end 181.783621 138.603621) (width 0.5) (layer B.Cu) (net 6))
 (segment (start 181.783621 138.603621) (end 188.496305 138.603621) (width 0.5) (layer B.Cu) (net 6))
 (segment (start 188.496305 138.603621) (end 190.63002 136.469906) (width 0.5) (layer B.Cu) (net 6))
 (segment (start 190.63002 136.469906) (end 190.63002 116.820418) (width 0.5) (layer B.Cu) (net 6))
 (segment (start 182.9736 114.054) (end 181.61 115.4176) (width 0.5) (layer B.Cu) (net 6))
 (segment (start 190.63002 116.820418) (end 187.863602 114.054) (width 0.5) (layer B.Cu) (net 6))
 (segment (start 181.61 115.4176) (end 181.61 115.57) (width 0.5) (layer B.Cu) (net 6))
 (segment (start 187.863602 114.054) (end 182.9736 114.054) (width 0.5) (layer B.Cu) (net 6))
 (segment (start 163.83 128.27) (end 163.83 133.35) (width 0.5) (layer B.Cu) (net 7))
 (segment (start 166.37 123.19) (end 166.37 123.040398) (width 0.5) (layer B.Cu) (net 8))
 (segment (start 166.37 123.040398) (end 165.053601 121.723999) (width 0.5) (layer B.Cu) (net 8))
 (segment (start 165.053601 121.723999) (end 162.606399 121.723999) (width 0.5) (layer B.Cu) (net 8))
 (segment (start 162.606399 121.723999) (end 161.816389 122.514009) (width 0.5) (layer B.Cu) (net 8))
 (segment (start 161.816389 122.514009) (end 161.816389 136.413591) (width 0.5) (layer B.Cu) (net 8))
 (segment (start 161.816389 136.413591) (end 162.606399 137.203601) (width 0.5) (layer B.Cu) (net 8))
 (segment (start 162.606399 137.203601) (end 165.056399 137.203601) (width 0.5) (layer B.Cu) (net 8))
 (segment (start 165.056399 137.203601) (end 165.506401 136.753599) (width 0.5) (layer B.Cu) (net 8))
 (segment (start 165.506401 136.753599) (end 166.37 135.89) (width 0.5) (layer B.Cu) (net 8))
 (segment (start 166.37 128.27) (end 166.37 133.35) (width 0.5) (layer B.Cu) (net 9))
 (segment (start 168.91 128.27) (end 168.91 133.35) (width 0.5) (layer B.Cu) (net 11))
 (segment (start 168.046401 136.753599) (end 168.91 135.89) (width 0.5) (layer B.Cu) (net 10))
 (segment (start 162.316446 137.903611) (end 166.896389 137.903611) (width 0.5) (layer B.Cu) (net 10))
 (segment (start 161.116379 136.703544) (end 162.316446 137.903611) (width 0.5) (layer B.Cu) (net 10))
 (segment (start 161.116379 122.224056) (end 161.116379 136.703544) (width 0.5) (layer B.Cu) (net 10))
 (segment (start 162.316446 121.023989) (end 161.116379 122.224056) (width 0.5) (layer B.Cu) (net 10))
 (segment (start 166.896389 121.023989) (end 162.316446 121.023989) (width 0.5) (layer B.Cu) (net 10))
 (segment (start 168.91 123.0376) (end 166.896389 121.023989) (width 0.5) (layer B.Cu) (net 10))
 (segment (start 166.896389 137.903611) (end 168.046401 136.753599) (width 0.5) (layer B.Cu) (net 10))
 (segment (start 168.91 123.19) (end 168.91 123.0376) (width 0.5) (layer B.Cu) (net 10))
 (segment (start 171.45 128.27) (end 171.45 133.35) (width 0.5) (layer B.Cu) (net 12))
 (segment (start 173.99 133.35) (end 173.99 126.190087) (width 0.5) (layer F.Cu) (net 13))
 (segment (start 173.99 126.190087) (end 173.155924 125.356011) (width 0.5) (layer F.Cu) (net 13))
 (segment (start 173.155924 125.356011) (end 162.316446 125.356011) (width 0.5) (layer F.Cu) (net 13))
 (segment (start 161.81638 107.274018) (end 162.656398 106.434) (width 0.5) (layer F.Cu) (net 13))
 (segment (start 184.15 107.7976) (end 184.15 107.95) (width 0.5) (layer F.Cu) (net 13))
 (segment (start 162.316446 125.356011) (end 161.81638 124.855945) (width 0.5) (layer F.Cu) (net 13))
 (segment (start 161.81638 124.855945) (end 161.81638 107.274018) (width 0.5) (layer F.Cu) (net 13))
 (segment (start 162.656398 106.434) (end 182.7864 106.434) (width 0.5) (layer F.Cu) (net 13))
 (segment (start 182.7864 106.434) (end 184.15 107.7976) (width 0.5) (layer F.Cu) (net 13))
 (segment (start 176.53 133.35) (end 176.53 127.740125) (width 0.5) (layer F.Cu) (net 14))
 (segment (start 176.53 127.740125) (end 173.445876 124.656001) (width 0.5) (layer F.Cu) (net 14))
 (segment (start 162.606399 124.656001) (end 162.51639 124.565992) (width 0.5) (layer F.Cu) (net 14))
 (segment (start 173.445876 124.656001) (end 162.606399 124.656001) (width 0.5) (layer F.Cu) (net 14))
 (segment (start 162.51639 124.565992) (end 162.51639 111.95601) (width 0.5) (layer F.Cu) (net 14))
 (segment (start 162.51639 111.95601) (end 166.37 108.1024) (width 0.5) (layer F.Cu) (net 14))
 (segment (start 166.37 108.1024) (end 166.37 107.95) (width 0.5) (layer F.Cu) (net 14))
 (segment (start 179.07 133.35) (end 188.00361 124.41639) (width 0.5) (layer F.Cu) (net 15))
 (segment (start 188.00361 124.41639) (end 188.00361 122.493485) (width 0.5) (layer F.Cu) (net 15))
 (segment (start 188.00361 122.493485) (end 182.546135 117.03601) (width 0.5) (layer F.Cu) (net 15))
 (segment (start 182.546135 117.03601) (end 178.525885 117.03601) (width 0.5) (layer F.Cu) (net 15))
 (segment (start 178.525885 117.03601) (end 176.53 115.040125) (width 0.5) (layer F.Cu) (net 15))
 (segment (start 176.53 109.466) (end 176.53 107.95) (width 0.5) (layer F.Cu) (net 15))
 (segment (start 176.53 115.040125) (end 176.53 109.466) (width 0.5) (layer F.Cu) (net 15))
 (segment (start 181.61 133.35) (end 181.61 130.81) (width 0.5) (layer B.Cu) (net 16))
 (segment (start 173.99 123.3424) (end 173.99 123.19) (width 0.5) (layer B.Cu) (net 16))
 (segment (start 181.61 130.81) (end 175.506 124.706) (width 0.5) (layer B.Cu) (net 16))
 (segment (start 175.506 124.706) (end 175.3536 124.706) (width 0.5) (layer B.Cu) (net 16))
 (segment (start 175.3536 124.706) (end 173.99 123.3424) (width 0.5) (layer B.Cu) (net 16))
 (segment (start 184.15 123.19) (end 184.15 124.706) (width 0.5) (layer B.Cu) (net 17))
 (segment (start 189.23 135.89) (end 187.916399 137.203601) (width 0.5) (layer B.Cu) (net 17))
 (segment (start 184.15 124.706) (end 189.23 129.786) (width 0.5) (layer B.Cu) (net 17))
 (segment (start 189.23 129.786) (end 189.23 135.89) (width 0.5) (layer B.Cu) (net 17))
 (segment (start 187.916399 137.203601) (end 185.463601 137.203601) (width 0.5) (layer B.Cu) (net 17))
 (segment (start 185.463601 137.203601) (end 185.013599 136.753599) (width 0.5) (layer B.Cu) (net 17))
 (segment (start 185.013599 136.753599) (end 184.15 135.89) (width 0.5) (layer B.Cu) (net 17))
 (segment (start 184.15 133.35) (end 184.15 130.81) (width 0.5) (layer B.Cu) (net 18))
 (segment (start 176.53 123.3424) (end 176.53 123.19) (width 0.5) (layer B.Cu) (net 18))
 (segment (start 184.15 130.81) (end 178.046 124.706) (width 0.5) (layer B.Cu) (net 18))
 (segment (start 178.046 124.706) (end 177.8936 124.706) (width 0.5) (layer B.Cu) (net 18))
 (segment (start 177.8936 124.706) (end 176.53 123.3424) (width 0.5) (layer B.Cu) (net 18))
 (segment (start 181.61 123.19) (end 181.61 124.706) (width 0.5) (layer B.Cu) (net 19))
 (segment (start 181.61 124.706) (end 188.003601 131.099601) (width 0.5) (layer B.Cu) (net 19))
 (segment (start 187.553599 135.026401) (end 186.69 135.89) (width 0.5) (layer B.Cu) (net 19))
 (segment (start 188.003601 131.099601) (end 188.003601 134.576399) (width 0.5) (layer B.Cu) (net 19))
 (segment (start 188.003601 134.576399) (end 187.553599 135.026401) (width 0.5) (layer B.Cu) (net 19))
 (segment (start 181.61 123.19) (end 181.61 123.0376) (width 0.5) (layer B.Cu) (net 19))
 (segment (start 186.69 133.35) (end 186.69 130.81) (width 0.5) (layer B.Cu) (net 20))
 (segment (start 186.69 130.81) (end 180.586 124.706) (width 0.5) (layer B.Cu) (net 20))
 (segment (start 180.586 124.706) (end 180.4336 124.706) (width 0.5) (layer B.Cu) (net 20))
 (segment (start 180.4336 124.706) (end 179.07 123.3424) (width 0.5) (layer B.Cu) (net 20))
 (segment (start 179.07 123.3424) (end 179.07 123.19) (width 0.5) (layer B.Cu) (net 20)))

